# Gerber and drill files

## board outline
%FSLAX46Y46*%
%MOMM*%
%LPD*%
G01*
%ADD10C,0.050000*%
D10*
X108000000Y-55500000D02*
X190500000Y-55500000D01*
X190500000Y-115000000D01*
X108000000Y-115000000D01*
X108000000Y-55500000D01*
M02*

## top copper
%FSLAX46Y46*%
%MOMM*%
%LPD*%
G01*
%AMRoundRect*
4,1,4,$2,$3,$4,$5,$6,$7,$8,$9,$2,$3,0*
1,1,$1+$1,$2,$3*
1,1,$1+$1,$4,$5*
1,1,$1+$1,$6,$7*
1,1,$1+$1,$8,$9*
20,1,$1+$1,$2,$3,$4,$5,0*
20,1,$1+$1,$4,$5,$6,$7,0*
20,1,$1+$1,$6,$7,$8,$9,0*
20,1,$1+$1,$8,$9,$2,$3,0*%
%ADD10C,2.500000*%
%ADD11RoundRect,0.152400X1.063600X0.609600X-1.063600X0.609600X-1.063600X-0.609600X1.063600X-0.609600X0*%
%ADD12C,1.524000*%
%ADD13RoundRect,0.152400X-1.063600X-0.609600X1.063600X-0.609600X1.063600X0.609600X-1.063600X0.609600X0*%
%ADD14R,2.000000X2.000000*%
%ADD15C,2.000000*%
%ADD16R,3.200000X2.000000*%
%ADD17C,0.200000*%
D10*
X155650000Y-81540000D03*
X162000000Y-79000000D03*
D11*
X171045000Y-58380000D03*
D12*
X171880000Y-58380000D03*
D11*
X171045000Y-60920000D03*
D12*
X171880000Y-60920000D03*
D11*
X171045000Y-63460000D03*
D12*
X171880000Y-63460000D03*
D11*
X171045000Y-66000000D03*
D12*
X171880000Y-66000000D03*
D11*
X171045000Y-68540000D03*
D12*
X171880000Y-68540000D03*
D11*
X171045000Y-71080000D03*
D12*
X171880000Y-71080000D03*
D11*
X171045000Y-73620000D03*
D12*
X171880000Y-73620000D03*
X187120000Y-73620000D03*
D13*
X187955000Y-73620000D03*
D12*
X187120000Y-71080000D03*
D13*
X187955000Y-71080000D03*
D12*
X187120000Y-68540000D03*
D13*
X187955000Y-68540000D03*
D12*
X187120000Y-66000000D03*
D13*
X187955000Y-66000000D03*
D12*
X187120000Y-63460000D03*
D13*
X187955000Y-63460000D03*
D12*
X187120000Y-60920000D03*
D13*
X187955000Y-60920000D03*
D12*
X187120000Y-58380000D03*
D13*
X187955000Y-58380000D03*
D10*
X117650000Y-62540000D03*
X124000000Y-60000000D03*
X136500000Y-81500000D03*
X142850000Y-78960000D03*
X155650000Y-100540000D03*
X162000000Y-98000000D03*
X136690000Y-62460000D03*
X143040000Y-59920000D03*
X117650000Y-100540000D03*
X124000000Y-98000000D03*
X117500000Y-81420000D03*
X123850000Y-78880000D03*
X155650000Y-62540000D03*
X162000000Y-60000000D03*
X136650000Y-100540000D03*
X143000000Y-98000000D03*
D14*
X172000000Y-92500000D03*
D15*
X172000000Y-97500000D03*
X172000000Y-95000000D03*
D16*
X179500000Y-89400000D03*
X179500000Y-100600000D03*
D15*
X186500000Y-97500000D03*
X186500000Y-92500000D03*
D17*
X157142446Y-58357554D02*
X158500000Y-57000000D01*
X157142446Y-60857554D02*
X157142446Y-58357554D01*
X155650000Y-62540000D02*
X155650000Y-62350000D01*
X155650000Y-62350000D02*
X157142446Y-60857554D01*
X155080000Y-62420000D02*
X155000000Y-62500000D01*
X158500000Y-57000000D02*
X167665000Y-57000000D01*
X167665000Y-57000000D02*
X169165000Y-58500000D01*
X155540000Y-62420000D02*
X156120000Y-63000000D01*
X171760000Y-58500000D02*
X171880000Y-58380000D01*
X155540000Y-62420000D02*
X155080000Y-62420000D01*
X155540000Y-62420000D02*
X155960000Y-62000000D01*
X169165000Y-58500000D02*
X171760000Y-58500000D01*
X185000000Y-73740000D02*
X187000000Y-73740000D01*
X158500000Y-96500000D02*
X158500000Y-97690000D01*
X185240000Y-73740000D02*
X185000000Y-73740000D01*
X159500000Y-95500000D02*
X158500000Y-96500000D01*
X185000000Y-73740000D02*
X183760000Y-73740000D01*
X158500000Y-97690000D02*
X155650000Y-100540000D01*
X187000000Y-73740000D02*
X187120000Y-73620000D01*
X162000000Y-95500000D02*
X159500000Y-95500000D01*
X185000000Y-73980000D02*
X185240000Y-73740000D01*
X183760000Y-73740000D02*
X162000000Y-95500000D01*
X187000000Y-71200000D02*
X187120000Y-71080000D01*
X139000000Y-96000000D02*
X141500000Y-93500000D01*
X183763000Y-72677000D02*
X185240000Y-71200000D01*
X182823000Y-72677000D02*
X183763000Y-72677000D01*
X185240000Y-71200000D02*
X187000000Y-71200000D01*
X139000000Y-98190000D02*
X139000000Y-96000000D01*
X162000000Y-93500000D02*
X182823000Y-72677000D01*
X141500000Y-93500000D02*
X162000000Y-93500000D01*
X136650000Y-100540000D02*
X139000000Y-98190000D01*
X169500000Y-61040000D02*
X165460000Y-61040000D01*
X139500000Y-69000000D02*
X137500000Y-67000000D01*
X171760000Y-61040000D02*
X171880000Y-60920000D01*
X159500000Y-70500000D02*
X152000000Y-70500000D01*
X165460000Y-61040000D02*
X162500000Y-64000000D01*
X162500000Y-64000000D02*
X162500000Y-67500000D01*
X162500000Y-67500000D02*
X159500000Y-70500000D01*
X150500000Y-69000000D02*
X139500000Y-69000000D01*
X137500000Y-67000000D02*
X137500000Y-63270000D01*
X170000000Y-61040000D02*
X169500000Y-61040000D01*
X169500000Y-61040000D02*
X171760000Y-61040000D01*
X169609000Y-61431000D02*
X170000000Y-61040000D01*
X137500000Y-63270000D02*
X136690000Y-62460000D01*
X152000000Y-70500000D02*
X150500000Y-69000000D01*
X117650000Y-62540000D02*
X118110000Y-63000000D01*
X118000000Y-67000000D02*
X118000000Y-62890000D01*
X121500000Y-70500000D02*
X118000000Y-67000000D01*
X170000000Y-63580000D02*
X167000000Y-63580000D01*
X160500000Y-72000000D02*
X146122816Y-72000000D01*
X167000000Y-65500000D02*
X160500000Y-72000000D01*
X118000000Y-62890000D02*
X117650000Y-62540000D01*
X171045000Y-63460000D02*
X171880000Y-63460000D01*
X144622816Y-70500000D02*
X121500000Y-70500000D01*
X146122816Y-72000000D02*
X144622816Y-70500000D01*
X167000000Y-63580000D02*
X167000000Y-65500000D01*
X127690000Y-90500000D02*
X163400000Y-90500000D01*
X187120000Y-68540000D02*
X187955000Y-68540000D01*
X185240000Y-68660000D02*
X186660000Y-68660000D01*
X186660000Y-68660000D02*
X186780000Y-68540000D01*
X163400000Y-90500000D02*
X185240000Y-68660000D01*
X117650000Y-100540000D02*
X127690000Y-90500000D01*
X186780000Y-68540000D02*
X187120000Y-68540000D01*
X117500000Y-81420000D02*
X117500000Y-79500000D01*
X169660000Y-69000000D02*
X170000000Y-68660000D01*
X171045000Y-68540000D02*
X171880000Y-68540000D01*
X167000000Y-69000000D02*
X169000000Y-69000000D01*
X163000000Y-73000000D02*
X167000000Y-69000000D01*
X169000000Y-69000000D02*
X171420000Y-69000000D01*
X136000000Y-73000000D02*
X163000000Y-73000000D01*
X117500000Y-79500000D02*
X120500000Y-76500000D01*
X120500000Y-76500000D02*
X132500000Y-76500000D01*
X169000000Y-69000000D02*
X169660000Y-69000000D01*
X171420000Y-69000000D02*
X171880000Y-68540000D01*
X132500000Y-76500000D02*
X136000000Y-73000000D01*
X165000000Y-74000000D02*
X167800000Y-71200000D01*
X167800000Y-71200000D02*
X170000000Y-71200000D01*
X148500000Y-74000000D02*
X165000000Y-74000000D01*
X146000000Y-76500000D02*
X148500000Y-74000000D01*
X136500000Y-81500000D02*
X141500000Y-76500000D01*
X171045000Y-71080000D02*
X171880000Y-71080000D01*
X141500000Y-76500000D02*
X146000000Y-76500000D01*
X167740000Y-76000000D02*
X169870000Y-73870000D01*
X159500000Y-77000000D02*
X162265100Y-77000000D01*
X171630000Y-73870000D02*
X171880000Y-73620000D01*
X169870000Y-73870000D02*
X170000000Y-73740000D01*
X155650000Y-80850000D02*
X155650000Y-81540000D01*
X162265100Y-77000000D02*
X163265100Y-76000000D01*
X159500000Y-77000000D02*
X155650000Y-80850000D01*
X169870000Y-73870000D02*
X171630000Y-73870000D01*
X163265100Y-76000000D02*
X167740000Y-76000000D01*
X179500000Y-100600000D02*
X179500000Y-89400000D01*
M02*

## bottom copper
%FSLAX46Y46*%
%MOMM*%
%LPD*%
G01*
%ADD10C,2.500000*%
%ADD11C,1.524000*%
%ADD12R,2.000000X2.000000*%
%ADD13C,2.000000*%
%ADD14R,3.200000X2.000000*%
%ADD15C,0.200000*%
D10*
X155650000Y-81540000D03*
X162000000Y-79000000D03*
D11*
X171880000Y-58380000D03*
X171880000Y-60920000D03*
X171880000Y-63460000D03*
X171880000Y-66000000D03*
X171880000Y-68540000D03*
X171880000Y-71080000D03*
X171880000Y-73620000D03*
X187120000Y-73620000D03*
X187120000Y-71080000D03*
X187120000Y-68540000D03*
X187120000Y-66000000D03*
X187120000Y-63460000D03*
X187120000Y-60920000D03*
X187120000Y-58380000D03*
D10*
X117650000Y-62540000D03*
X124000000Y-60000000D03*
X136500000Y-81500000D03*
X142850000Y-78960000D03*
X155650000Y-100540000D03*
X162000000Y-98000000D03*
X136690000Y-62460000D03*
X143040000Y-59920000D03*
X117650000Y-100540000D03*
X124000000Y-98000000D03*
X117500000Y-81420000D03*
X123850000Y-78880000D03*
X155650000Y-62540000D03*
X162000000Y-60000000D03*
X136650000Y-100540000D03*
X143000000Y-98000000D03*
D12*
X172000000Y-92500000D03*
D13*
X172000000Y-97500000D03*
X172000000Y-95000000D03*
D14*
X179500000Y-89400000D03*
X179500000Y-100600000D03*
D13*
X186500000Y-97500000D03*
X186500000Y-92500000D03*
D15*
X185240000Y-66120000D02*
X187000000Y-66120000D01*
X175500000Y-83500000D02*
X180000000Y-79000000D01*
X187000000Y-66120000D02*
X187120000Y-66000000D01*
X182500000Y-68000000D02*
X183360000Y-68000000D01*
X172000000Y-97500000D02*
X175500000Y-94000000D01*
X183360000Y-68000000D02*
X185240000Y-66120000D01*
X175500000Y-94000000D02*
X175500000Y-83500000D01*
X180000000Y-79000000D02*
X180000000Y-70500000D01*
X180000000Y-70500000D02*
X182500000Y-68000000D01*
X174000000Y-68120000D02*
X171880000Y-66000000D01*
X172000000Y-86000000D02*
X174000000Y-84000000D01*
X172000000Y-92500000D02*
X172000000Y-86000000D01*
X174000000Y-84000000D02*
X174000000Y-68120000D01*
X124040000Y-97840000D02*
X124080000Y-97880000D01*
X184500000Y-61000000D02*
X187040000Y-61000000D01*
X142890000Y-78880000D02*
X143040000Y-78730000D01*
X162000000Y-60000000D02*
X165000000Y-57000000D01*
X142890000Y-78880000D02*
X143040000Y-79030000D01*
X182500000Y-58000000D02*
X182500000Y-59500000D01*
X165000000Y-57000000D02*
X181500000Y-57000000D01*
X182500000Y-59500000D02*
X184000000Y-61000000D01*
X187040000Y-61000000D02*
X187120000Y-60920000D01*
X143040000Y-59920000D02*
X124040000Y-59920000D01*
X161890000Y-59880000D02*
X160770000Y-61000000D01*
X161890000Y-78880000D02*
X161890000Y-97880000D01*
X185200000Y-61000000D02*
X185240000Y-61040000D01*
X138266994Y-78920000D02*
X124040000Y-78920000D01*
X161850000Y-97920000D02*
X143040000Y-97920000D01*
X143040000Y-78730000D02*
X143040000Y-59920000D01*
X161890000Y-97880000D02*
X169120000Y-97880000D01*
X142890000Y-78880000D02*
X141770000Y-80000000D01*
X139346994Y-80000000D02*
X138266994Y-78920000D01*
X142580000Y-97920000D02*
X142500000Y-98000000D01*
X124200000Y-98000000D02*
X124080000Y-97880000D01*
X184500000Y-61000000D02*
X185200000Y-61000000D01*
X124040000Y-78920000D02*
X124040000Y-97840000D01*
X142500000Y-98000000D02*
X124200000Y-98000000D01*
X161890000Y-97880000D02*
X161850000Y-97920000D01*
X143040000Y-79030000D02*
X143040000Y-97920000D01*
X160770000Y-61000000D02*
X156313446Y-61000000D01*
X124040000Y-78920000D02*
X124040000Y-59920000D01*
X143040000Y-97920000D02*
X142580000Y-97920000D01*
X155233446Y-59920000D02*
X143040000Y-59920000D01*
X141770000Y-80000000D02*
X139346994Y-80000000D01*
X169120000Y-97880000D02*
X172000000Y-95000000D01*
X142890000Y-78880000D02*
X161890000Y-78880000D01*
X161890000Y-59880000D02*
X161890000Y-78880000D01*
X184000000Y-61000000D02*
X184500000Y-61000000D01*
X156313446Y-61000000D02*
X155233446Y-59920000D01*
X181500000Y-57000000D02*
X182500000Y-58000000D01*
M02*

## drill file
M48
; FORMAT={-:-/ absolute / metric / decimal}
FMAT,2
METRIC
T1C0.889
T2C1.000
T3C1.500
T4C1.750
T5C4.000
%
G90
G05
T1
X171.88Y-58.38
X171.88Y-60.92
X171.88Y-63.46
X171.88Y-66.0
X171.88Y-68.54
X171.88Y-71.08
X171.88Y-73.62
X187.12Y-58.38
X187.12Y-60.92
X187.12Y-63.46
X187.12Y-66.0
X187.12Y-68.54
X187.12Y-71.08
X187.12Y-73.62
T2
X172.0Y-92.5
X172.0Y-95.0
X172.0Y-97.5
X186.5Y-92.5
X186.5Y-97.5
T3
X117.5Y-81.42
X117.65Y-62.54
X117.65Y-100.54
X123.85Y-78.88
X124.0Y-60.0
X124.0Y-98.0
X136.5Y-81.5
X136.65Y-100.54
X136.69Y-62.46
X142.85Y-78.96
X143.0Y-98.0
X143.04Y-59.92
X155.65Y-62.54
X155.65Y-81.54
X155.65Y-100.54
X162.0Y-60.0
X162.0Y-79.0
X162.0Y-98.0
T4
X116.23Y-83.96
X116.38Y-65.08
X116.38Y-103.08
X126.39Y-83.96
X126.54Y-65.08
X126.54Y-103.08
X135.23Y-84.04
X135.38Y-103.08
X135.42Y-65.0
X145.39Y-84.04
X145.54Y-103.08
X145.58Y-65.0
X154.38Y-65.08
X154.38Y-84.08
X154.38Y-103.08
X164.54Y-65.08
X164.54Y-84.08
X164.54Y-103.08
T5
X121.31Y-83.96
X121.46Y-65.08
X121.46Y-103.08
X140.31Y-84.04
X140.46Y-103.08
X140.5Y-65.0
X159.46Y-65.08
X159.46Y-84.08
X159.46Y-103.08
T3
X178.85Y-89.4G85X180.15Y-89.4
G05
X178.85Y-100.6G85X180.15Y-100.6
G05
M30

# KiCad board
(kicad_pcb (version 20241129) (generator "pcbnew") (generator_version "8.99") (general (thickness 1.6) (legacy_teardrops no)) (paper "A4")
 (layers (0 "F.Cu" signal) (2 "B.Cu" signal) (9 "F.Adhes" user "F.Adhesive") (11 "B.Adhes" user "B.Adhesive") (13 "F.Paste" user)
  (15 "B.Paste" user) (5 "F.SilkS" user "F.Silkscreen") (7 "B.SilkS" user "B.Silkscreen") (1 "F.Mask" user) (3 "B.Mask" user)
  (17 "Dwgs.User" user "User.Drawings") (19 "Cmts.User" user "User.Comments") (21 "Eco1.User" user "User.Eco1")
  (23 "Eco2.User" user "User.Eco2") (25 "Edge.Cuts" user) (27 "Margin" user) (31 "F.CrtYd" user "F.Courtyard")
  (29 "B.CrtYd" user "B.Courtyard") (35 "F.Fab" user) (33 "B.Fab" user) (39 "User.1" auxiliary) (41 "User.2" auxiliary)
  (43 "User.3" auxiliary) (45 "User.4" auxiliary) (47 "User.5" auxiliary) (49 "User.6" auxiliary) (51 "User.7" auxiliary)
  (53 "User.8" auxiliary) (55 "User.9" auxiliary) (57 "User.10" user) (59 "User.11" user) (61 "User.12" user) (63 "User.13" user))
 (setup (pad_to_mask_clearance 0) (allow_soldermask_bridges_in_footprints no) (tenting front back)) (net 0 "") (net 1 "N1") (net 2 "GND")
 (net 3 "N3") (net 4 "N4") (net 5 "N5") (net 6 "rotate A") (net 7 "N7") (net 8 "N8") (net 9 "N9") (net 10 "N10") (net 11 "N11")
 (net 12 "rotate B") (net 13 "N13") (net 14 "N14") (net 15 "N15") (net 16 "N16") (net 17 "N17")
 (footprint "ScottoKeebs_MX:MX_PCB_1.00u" (layer "F.Cu") (at 159.46 84.08)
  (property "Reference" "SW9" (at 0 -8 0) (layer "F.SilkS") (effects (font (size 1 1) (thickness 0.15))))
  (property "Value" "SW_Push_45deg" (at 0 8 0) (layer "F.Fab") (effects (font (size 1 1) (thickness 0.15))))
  (pad "" np_thru_hole circle (at -5.08 0) (size 1.75 1.75) (drill 1.75) (layers "*.Cu" "*.Mask"))
  (pad "" np_thru_hole circle (at 0 0) (size 4 4) (drill 4) (layers "*.Cu" "*.Mask"))
  (pad "" np_thru_hole circle (at 5.08 0) (size 1.75 1.75) (drill 1.75) (layers "*.Cu" "*.Mask"))
  (pad "1" thru_hole circle (at -3.81 -2.54) (size 2.5 2.5) (drill 1.5) (layers "*.Cu" "*.Mask") (remove_unused_layers no) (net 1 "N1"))
  (pad "2" thru_hole circle (at 2.54 -5.08) (size 2.5 2.5) (drill 1.5) (layers "*.Cu" "*.Mask") (remove_unused_layers no) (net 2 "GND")))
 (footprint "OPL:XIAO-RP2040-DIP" (layer "F.Cu") (at 179.5 66)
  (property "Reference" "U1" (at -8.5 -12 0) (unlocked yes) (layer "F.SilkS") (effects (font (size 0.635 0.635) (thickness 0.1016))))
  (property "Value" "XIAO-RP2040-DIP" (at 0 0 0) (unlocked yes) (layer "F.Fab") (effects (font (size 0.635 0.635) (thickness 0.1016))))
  (pad "1" smd roundrect (at -8.455 -7.62 180) (size 2.432 1.524) (layers "F.Cu" "F.Mask") (roundrect_rratio 0.1) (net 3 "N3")
   (thermal_bridge_angle 45))
  (pad "1" thru_hole circle (at -7.62 -7.62 180) (size 1.524 1.524) (drill 0.889) (layers "*.Cu" "*.Mask") (remove_unused_layers no)
   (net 3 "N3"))
  (pad "2" smd roundrect (at -8.455 -5.08 180) (size 2.432 1.524) (layers "F.Cu" "F.Mask") (roundrect_rratio 0.1) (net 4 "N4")
   (thermal_bridge_angle 45))
  (pad "2" thru_hole circle (at -7.62 -5.08 180) (size 1.524 1.524) (drill 0.889) (layers "*.Cu" "*.Mask") (remove_unused_layers no)
   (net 4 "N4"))
  (pad "3" smd roundrect (at -8.455 -2.54 180) (size 2.432 1.524) (layers "F.Cu" "F.Mask") (roundrect_rratio 0.1) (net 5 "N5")
   (thermal_bridge_angle 45))
  (pad "3" thru_hole circle (at -7.62 -2.54 180) (size 1.524 1.524) (drill 0.889) (layers "*.Cu" "*.Mask") (remove_unused_layers no)
   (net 5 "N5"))
  (pad "4" smd roundrect (at -8.455 0 180) (size 2.432 1.524) (layers "F.Cu" "F.Mask") (roundrect_rratio 0.1) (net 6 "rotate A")
   (thermal_bridge_angle 45))
  (pad "4" thru_hole circle (at -7.62 0 180) (size 1.524 1.524) (drill 0.889) (layers "*.Cu" "*.Mask") (remove_unused_layers no)
   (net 6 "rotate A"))
  (pad "5" smd roundrect (at -8.455 2.54 180) (size 2.432 1.524) (layers "F.Cu" "F.Mask") (roundrect_rratio 0.1) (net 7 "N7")
   (thermal_bridge_angle 45))
  (pad "5" thru_hole circle (at -7.62 2.54 180) (size 1.524 1.524) (drill 0.889) (layers "*.Cu" "*.Mask") (remove_unused_layers no)
   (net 7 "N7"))
  (pad "6" smd roundrect (at -8.455 5.08 180) (size 2.432 1.524) (layers "F.Cu" "F.Mask") (roundrect_rratio 0.1) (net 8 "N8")
   (thermal_bridge_angle 45))
  (pad "6" thru_hole circle (at -7.62 5.08 180) (size 1.524 1.524) (drill 0.889) (layers "*.Cu" "*.Mask") (remove_unused_layers no)
   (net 8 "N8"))
  (pad "7" smd roundrect (at -8.455 7.62 180) (size 2.432 1.524) (layers "F.Cu" "F.Mask") (roundrect_rratio 0.1) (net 1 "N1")
   (thermal_bridge_angle 45))
  (pad "7" thru_hole circle (at -7.62 7.62 180) (size 1.524 1.524) (drill 0.889) (layers "*.Cu" "*.Mask") (remove_unused_layers no)
   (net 1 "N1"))
  (pad "8" thru_hole circle (at 7.62 7.62) (size 1.524 1.524) (drill 0.889) (layers "*.Cu" "*.Mask") (remove_unused_layers no) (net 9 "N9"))
  (pad "8" smd roundrect (at 8.455 7.62) (size 2.432 1.524) (layers "F.Cu" "F.Mask") (roundrect_rratio 0.1) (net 9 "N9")
   (thermal_bridge_angle 45))
  (pad "9" thru_hole circle (at 7.62 5.08) (size 1.524 1.524) (drill 0.889) (layers "*.Cu" "*.Mask") (remove_unused_layers no)
   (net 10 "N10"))
  (pad "9" smd roundrect (at 8.455 5.08) (size 2.432 1.524) (layers "F.Cu" "F.Mask") (roundrect_rratio 0.1) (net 10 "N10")
   (thermal_bridge_angle 45))
  (pad "10" thru_hole circle (at 7.62 2.54) (size 1.524 1.524) (drill 0.889) (layers "*.Cu" "*.Mask") (remove_unused_layers no)
   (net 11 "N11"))
  (pad "10" smd roundrect (at 8.455 2.54) (size 2.432 1.524) (layers "F.Cu" "F.Mask") (roundrect_rratio 0.1) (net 11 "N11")
   (thermal_bridge_angle 45))
  (pad "11" thru_hole circle (at 7.62 0) (size 1.524 1.524) (drill 0.889) (layers "*.Cu" "*.Mask") (remove_unused_layers no)
   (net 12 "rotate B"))
  (pad "11" smd roundrect (at 8.455 0) (size 2.432 1.524) (layers "F.Cu" "F.Mask") (roundrect_rratio 0.1) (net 12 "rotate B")
   (thermal_bridge_angle 45))
  (pad "12" thru_hole circle (at 7.62 -2.54) (size 1.524 1.524) (drill 0.889) (layers "*.Cu" "*.Mask") (remove_unused_layers no)
   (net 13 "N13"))
  (pad "12" smd roundrect (at 8.455 -2.54) (size 2.432 1.524) (layers "F.Cu" "F.Mask") (roundrect_rratio 0.1) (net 13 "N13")
   (thermal_bridge_angle 45))
  (pad "13" thru_hole circle (at 7.62 -5.08) (size 1.524 1.524) (drill 0.889) (layers "*.Cu" "*.Mask") (remove_unused_layers no)
   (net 2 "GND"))
  (pad "13" smd roundrect (at 8.455 -5.08) (size 2.432 1.524) (layers "F.Cu" "F.Mask") (roundrect_rratio 0.1) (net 2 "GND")
   (thermal_bridge_angle 45))
  (pad "14" thru_hole circle (at 7.62 -7.62) (size 1.524 1.524) (drill 0.889) (layers "*.Cu" "*.Mask") (remove_unused_layers no)
   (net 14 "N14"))
  (pad "14" smd roundrect (at 8.455 -7.62) (size 2.432 1.524) (layers "F.Cu" "F.Mask") (roundrect_rratio 0.1) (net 14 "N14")
   (thermal_bridge_angle 45)))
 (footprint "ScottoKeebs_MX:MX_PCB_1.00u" (layer "F.Cu") (at 121.46 65.08)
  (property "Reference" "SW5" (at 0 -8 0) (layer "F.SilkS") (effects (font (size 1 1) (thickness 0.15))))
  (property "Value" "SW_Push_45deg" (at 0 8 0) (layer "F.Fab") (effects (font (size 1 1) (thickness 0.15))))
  (pad "" np_thru_hole circle (at -5.08 0) (size 1.75 1.75) (drill 1.75) (layers "*.Cu" "*.Mask"))
  (pad "" np_thru_hole circle (at 0 0) (size 4 4) (drill 4) (layers "*.Cu" "*.Mask"))
  (pad "" np_thru_hole circle (at 5.08 0) (size 1.75 1.75) (drill 1.75) (layers "*.Cu" "*.Mask"))
  (pad "1" thru_hole circle (at -3.81 -2.54) (size 2.5 2.5) (drill 1.5) (layers "*.Cu" "*.Mask") (remove_unused_layers no) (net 5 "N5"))
  (pad "2" thru_hole circle (at 2.54 -5.08) (size 2.5 2.5) (drill 1.5) (layers "*.Cu" "*.Mask") (remove_unused_layers no) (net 2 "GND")))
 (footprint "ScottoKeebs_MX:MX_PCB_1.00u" (layer "F.Cu") (at 140.31 84.04)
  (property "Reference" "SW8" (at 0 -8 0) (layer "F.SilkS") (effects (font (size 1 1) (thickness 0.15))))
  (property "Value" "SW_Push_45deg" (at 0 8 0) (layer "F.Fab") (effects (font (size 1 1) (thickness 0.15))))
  (pad "" np_thru_hole circle (at -5.08 0) (size 1.75 1.75) (drill 1.75) (layers "*.Cu" "*.Mask"))
  (pad "" np_thru_hole circle (at 0 0) (size 4 4) (drill 4) (layers "*.Cu" "*.Mask"))
  (pad "" np_thru_hole circle (at 5.08 0) (size 1.75 1.75) (drill 1.75) (layers "*.Cu" "*.Mask"))
  (pad "1" thru_hole circle (at -3.81 -2.54) (size 2.5 2.5) (drill 1.5) (layers "*.Cu" "*.Mask") (remove_unused_layers no) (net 8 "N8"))
  (pad "2" thru_hole circle (at 2.54 -5.08) (size 2.5 2.5) (drill 1.5) (layers "*.Cu" "*.Mask") (remove_unused_layers no) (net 2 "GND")))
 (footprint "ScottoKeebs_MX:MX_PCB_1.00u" (layer "F.Cu") (at 159.46 103.08)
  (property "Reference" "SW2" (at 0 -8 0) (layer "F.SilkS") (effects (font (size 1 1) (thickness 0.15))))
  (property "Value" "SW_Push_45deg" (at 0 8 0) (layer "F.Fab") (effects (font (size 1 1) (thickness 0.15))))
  (pad "" np_thru_hole circle (at -5.08 0) (size 1.75 1.75) (drill 1.75) (layers "*.Cu" "*.Mask"))
  (pad "" np_thru_hole circle (at 0 0) (size 4 4) (drill 4) (layers "*.Cu" "*.Mask"))
  (pad "" np_thru_hole circle (at 5.08 0) (size 1.75 1.75) (drill 1.75) (layers "*.Cu" "*.Mask"))
  (pad "1" thru_hole circle (at -3.81 -2.54) (size 2.5 2.5) (drill 1.5) (layers "*.Cu" "*.Mask") (remove_unused_layers no) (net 9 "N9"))
  (pad "2" thru_hole circle (at 2.54 -5.08) (size 2.5 2.5) (drill 1.5) (layers "*.Cu" "*.Mask") (remove_unused_layers no) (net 2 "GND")))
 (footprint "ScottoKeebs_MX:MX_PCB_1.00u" (layer "F.Cu") (at 140.5 65)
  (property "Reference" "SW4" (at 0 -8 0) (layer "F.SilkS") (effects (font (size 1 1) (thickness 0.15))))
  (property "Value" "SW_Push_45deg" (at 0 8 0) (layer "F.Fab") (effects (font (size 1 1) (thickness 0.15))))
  (pad "" np_thru_hole circle (at -5.08 0) (size 1.75 1.75) (drill 1.75) (layers "*.Cu" "*.Mask"))
  (pad "" np_thru_hole circle (at 0 0) (size 4 4) (drill 4) (layers "*.Cu" "*.Mask"))
  (pad "" np_thru_hole circle (at 5.08 0) (size 1.75 1.75) (drill 1.75) (layers "*.Cu" "*.Mask"))
  (pad "1" thru_hole circle (at -3.81 -2.54) (size 2.5 2.5) (drill 1.5) (layers "*.Cu" "*.Mask") (remove_unused_layers no) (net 4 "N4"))
  (pad "2" thru_hole circle (at 2.54 -5.08) (size 2.5 2.5) (drill 1.5) (layers "*.Cu" "*.Mask") (remove_unused_layers no) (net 2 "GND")))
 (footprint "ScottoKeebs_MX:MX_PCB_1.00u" (layer "F.Cu") (at 121.46 103.08)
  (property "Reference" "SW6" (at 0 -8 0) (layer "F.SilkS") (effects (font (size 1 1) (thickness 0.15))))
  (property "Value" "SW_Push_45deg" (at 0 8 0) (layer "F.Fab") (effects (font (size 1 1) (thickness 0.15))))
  (pad "" np_thru_hole circle (at -5.08 0) (size 1.75 1.75) (drill 1.75) (layers "*.Cu" "*.Mask"))
  (pad "" np_thru_hole circle (at 0 0) (size 4 4) (drill 4) (layers "*.Cu" "*.Mask"))
  (pad "" np_thru_hole circle (at 5.08 0) (size 1.75 1.75) (drill 1.75) (layers "*.Cu" "*.Mask"))
  (pad "1" thru_hole circle (at -3.81 -2.54) (size 2.5 2.5) (drill 1.5) (layers "*.Cu" "*.Mask") (remove_unused_layers no) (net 11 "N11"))
  (pad "2" thru_hole circle (at 2.54 -5.08) (size 2.5 2.5) (drill 1.5) (layers "*.Cu" "*.Mask") (remove_unused_layers no) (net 2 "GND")))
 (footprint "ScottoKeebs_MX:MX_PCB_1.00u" (layer "F.Cu") (at 121.31 83.96)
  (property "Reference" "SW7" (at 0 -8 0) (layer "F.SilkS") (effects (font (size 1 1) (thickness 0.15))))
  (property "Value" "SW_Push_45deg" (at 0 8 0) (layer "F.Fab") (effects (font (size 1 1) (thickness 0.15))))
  (pad "" np_thru_hole circle (at -5.08 0) (size 1.75 1.75) (drill 1.75) (layers "*.Cu" "*.Mask"))
  (pad "" np_thru_hole circle (at 0 0) (size 4 4) (drill 4) (layers "*.Cu" "*.Mask"))
  (pad "" np_thru_hole circle (at 5.08 0) (size 1.75 1.75) (drill 1.75) (layers "*.Cu" "*.Mask"))
  (pad "1" thru_hole circle (at -3.81 -2.54) (size 2.5 2.5) (drill 1.5) (layers "*.Cu" "*.Mask") (remove_unused_layers no) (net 7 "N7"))
  (pad "2" thru_hole circle (at 2.54 -5.08) (size 2.5 2.5) (drill 1.5) (layers "*.Cu" "*.Mask") (remove_unused_layers no) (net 2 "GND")))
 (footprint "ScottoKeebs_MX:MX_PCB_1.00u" (layer "F.Cu") (at 159.46 65.08)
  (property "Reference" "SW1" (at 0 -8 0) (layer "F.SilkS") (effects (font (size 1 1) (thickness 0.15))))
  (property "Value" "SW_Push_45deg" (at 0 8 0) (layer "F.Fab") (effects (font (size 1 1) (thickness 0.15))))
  (pad "" np_thru_hole circle (at -5.08 0) (size 1.75 1.75) (drill 1.75) (layers "*.Cu" "*.Mask"))
  (pad "" np_thru_hole circle (at 0 0) (size 4 4) (drill 4) (layers "*.Cu" "*.Mask"))
  (pad "" np_thru_hole circle (at 5.08 0) (size 1.75 1.75) (drill 1.75) (layers "*.Cu" "*.Mask"))
  (pad "1" thru_hole circle (at -3.81 -2.54) (size 2.5 2.5) (drill 1.5) (layers "*.Cu" "*.Mask") (remove_unused_layers no) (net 3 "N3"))
  (pad "2" thru_hole circle (at 2.54 -5.08) (size 2.5 2.5) (drill 1.5) (layers "*.Cu" "*.Mask") (remove_unused_layers no) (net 2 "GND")))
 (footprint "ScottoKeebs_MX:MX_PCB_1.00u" (layer "F.Cu") (at 140.46 103.08)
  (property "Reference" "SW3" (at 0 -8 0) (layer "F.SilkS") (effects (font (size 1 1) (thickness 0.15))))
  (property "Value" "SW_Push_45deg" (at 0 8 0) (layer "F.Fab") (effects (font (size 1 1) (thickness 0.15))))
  (pad "" np_thru_hole circle (at -5.08 0) (size 1.75 1.75) (drill 1.75) (layers "*.Cu" "*.Mask"))
  (pad "" np_thru_hole circle (at 0 0) (size 4 4) (drill 4) (layers "*.Cu" "*.Mask"))
  (pad "" np_thru_hole circle (at 5.08 0) (size 1.75 1.75) (drill 1.75) (layers "*.Cu" "*.Mask"))
  (pad "1" thru_hole circle (at -3.81 -2.54) (size 2.5 2.5) (drill 1.5) (layers "*.Cu" "*.Mask") (remove_unused_layers no) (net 10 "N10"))
  (pad "2" thru_hole circle (at 2.54 -5.08) (size 2.5 2.5) (drill 1.5) (layers "*.Cu" "*.Mask") (remove_unused_layers no) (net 2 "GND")))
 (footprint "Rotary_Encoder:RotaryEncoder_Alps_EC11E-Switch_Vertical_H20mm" (layer "F.Cu") (at 172 92.5)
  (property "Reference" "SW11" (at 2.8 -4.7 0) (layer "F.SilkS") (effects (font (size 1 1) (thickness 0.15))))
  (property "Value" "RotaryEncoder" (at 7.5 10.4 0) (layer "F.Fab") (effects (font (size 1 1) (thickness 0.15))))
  (pad "A" thru_hole rect (at 0 0) (size 2 2) (drill 1) (layers "*.Cu" "*.Mask") (remove_unused_layers no) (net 6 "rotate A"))
  (pad "B" thru_hole circle (at 0 5) (size 2 2) (drill 1) (layers "*.Cu" "*.Mask") (remove_unused_layers no) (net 12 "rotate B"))
  (pad "C" thru_hole circle (at 0 2.5) (size 2 2) (drill 1) (layers "*.Cu" "*.Mask") (remove_unused_layers no) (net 2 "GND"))
  (pad "MP" thru_hole rect (at 7.5 -3.1) (size 3.2 2) (drill oval 2.8 1.5) (layers "*.Cu" "*.Mask") (remove_unused_layers no) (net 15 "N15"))
  (pad "MP" thru_hole rect (at 7.5 8.1) (size 3.2 2) (drill oval 2.8 1.5) (layers "*.Cu" "*.Mask") (remove_unused_layers no) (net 15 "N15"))
  (pad "S1" thru_hole circle (at 14.5 5) (size 2 2) (drill 1) (layers "*.Cu" "*.Mask") (remove_unused_layers no) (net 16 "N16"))
  (pad "S2" thru_hole circle (at 14.5 0) (size 2 2) (drill 1) (layers "*.Cu" "*.Mask") (remove_unused_layers no) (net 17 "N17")))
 (gr_rect (start 108 55.5) (end 190.5 115) (stroke (width 0.05) (type default)) (fill no) (layer "Edge.Cuts"))
 (segment (start 157.142446 58.357554) (end 158.5 57) (width 0.2) (layer "F.Cu") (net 3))
 (segment (start 157.142446 60.857554) (end 157.142446 58.357554) (width 0.2) (layer "F.Cu") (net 3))
 (segment (start 155.65 62.54) (end 155.65 62.35) (width 0.2) (layer "F.Cu") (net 3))
 (segment (start 155.65 62.35) (end 157.142446 60.857554) (width 0.2) (layer "F.Cu") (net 3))
 (segment (start 155.08 62.42) (end 155 62.5) (width 0.2) (layer "F.Cu") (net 3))
 (segment (start 158.5 57) (end 167.665 57) (width 0.2) (layer "F.Cu") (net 3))
 (segment (start 167.665 57) (end 169.165 58.5) (width 0.2) (layer "F.Cu") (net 3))
 (segment (start 155.54 62.42) (end 156.12 63) (width 0.2) (layer "F.Cu") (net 3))
 (segment (start 171.76 58.5) (end 171.88 58.38) (width 0.2) (layer "F.Cu") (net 3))
 (segment (start 155.54 62.42) (end 155.08 62.42) (width 0.2) (layer "F.Cu") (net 3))
 (segment (start 155.54 62.42) (end 155.96 62) (width 0.2) (layer "F.Cu") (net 3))
 (segment (start 169.165 58.5) (end 171.76 58.5) (width 0.2) (layer "F.Cu") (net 3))
 (segment (start 185 73.74) (end 187 73.74) (width 0.2) (layer "F.Cu") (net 9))
 (segment (start 158.5 96.5) (end 158.5 97.69) (width 0.2) (layer "F.Cu") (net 9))
 (segment (start 185.24 73.74) (end 185 73.74) (width 0.2) (layer "F.Cu") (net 9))
 (segment (start 159.5 95.5) (end 158.5 96.5) (width 0.2) (layer "F.Cu") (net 9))
 (segment (start 185 73.74) (end 183.76 73.74) (width 0.2) (layer "F.Cu") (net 9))
 (segment (start 158.5 97.69) (end 155.65 100.54) (width 0.2) (layer "F.Cu") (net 9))
 (segment (start 187 73.74) (end 187.12 73.62) (width 0.2) (layer "F.Cu") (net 9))
 (segment (start 162 95.5) (end 159.5 95.5) (width 0.2) (layer "F.Cu") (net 9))
 (segment (start 185 73.98) (end 185.24 73.74) (width 0.2) (layer "F.Cu") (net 9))
 (segment (start 183.76 73.74) (end 162 95.5) (width 0.2) (layer "F.Cu") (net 9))
 (segment (start 187 71.2) (end 187.12 71.08) (width 0.2) (layer "F.Cu") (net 10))
 (segment (start 139 96) (end 141.5 93.5) (width 0.2) (layer "F.Cu") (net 10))
 (segment (start 183.763 72.677) (end 185.24 71.2) (width 0.2) (layer "F.Cu") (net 10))
 (segment (start 182.823 72.677) (end 183.763 72.677) (width 0.2) (layer "F.Cu") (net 10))
 (segment (start 185.24 71.2) (end 187 71.2) (width 0.2) (layer "F.Cu") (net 10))
 (segment (start 139 98.19) (end 139 96) (width 0.2) (layer "F.Cu") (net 10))
 (segment (start 162 93.5) (end 182.823 72.677) (width 0.2) (layer "F.Cu") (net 10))
 (segment (start 141.5 93.5) (end 162 93.5) (width 0.2) (layer "F.Cu") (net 10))
 (segment (start 136.65 100.54) (end 139 98.19) (width 0.2) (layer "F.Cu") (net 10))
 (segment (start 169.5 61.04) (end 165.46 61.04) (width 0.2) (layer "F.Cu") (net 4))
 (segment (start 139.5 69) (end 137.5 67) (width 0.2) (layer "F.Cu") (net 4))
 (segment (start 171.76 61.04) (end 171.88 60.92) (width 0.2) (layer "F.Cu") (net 4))
 (segment (start 159.5 70.5) (end 152 70.5) (width 0.2) (layer "F.Cu") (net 4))
 (segment (start 165.46 61.04) (end 162.5 64) (width 0.2) (layer "F.Cu") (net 4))
 (segment (start 162.5 64) (end 162.5 67.5) (width 0.2) (layer "F.Cu") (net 4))
 (segment (start 162.5 67.5) (end 159.5 70.5) (width 0.2) (layer "F.Cu") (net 4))
 (segment (start 150.5 69) (end 139.5 69) (width 0.2) (layer "F.Cu") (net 4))
 (segment (start 137.5 67) (end 137.5 63.27) (width 0.2) (layer "F.Cu") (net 4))
 (segment (start 170 61.04) (end 169.5 61.04) (width 0.2) (layer "F.Cu") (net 4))
 (segment (start 169.5 61.04) (end 171.76 61.04) (width 0.2) (layer "F.Cu") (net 4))
 (segment (start 169.609 61.431) (end 170 61.04) (width 0.2) (layer "F.Cu") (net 4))
 (segment (start 137.5 63.27) (end 136.69 62.46) (width 0.2) (layer "F.Cu") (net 4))
 (segment (start 152 70.5) (end 150.5 69) (width 0.2) (layer "F.Cu") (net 4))
 (segment (start 117.65 62.54) (end 118.11 63) (width 0.2) (layer "F.Cu") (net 5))
 (segment (start 118 67) (end 118 62.89) (width 0.2) (layer "F.Cu") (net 5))
 (segment (start 121.5 70.5) (end 118 67) (width 0.2) (layer "F.Cu") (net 5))
 (segment (start 170 63.58) (end 167 63.58) (width 0.2) (layer "F.Cu") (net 5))
 (segment (start 160.5 72) (end 146.122816 72) (width 0.2) (layer "F.Cu") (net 5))
 (segment (start 167 65.5) (end 160.5 72) (width 0.2) (layer "F.Cu") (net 5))
 (segment (start 118 62.89) (end 117.65 62.54) (width 0.2) (layer "F.Cu") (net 5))
 (segment (start 171.045 63.46) (end 171.88 63.46) (width 0.2) (layer "F.Cu") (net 5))
 (segment (start 144.622816 70.5) (end 121.5 70.5) (width 0.2) (layer "F.Cu") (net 5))
 (segment (start 146.122816 72) (end 144.622816 70.5) (width 0.2) (layer "F.Cu") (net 5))
 (segment (start 167 63.58) (end 167 65.5) (width 0.2) (layer "F.Cu") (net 5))
 (segment (start 127.69 90.5) (end 163.4 90.5) (width 0.2) (layer "F.Cu") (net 11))
 (segment (start 187.12 68.54) (end 187.955 68.54) (width 0.2) (layer "F.Cu") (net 11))
 (segment (start 185.24 68.66) (end 186.66 68.66) (width 0.2) (layer "F.Cu") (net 11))
 (segment (start 186.66 68.66) (end 186.78 68.54) (width 0.2) (layer "F.Cu") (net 11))
 (segment (start 163.4 90.5) (end 185.24 68.66) (width 0.2) (layer "F.Cu") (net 11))
 (segment (start 117.65 100.54) (end 127.69 90.5) (width 0.2) (layer "F.Cu") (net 11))
 (segment (start 186.78 68.54) (end 187.12 68.54) (width 0.2) (layer "F.Cu") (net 11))
 (segment (start 117.5 81.42) (end 117.5 79.5) (width 0.2) (layer "F.Cu") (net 7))
 (segment (start 169.66 69) (end 170 68.66) (width 0.2) (layer "F.Cu") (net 7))
 (segment (start 171.045 68.54) (end 171.88 68.54) (width 0.2) (layer "F.Cu") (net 7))
 (segment (start 167 69) (end 169 69) (width 0.2) (layer "F.Cu") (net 7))
 (segment (start 163 73) (end 167 69) (width 0.2) (layer "F.Cu") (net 7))
 (segment (start 169 69) (end 171.42 69) (width 0.2) (layer "F.Cu") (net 7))
 (segment (start 136 73) (end 163 73) (width 0.2) (layer "F.Cu") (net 7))
 (segment (start 117.5 79.5) (end 120.5 76.5) (width 0.2) (layer "F.Cu") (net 7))
 (segment (start 120.5 76.5) (end 132.5 76.5) (width 0.2) (layer "F.Cu") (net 7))
 (segment (start 169 69) (end 169.66 69) (width 0.2) (layer "F.Cu") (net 7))
 (segment (start 171.42 69) (end 171.88 68.54) (width 0.2) (layer "F.Cu") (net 7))
 (segment (start 132.5 76.5) (end 136 73) (width 0.2) (layer "F.Cu") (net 7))
 (segment (start 165 74) (end 167.8 71.2) (width 0.2) (layer "F.Cu") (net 8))
 (segment (start 167.8 71.2) (end 170 71.2) (width 0.2) (layer "F.Cu") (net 8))
 (segment (start 148.5 74) (end 165 74) (width 0.2) (layer "F.Cu") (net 8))
 (segment (start 146 76.5) (end 148.5 74) (width 0.2) (layer "F.Cu") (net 8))
 (segment (start 136.5 81.5) (end 141.5 76.5) (width 0.2) (layer "F.Cu") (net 8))
 (segment (start 171.045 71.08) (end 171.88 71.08) (width 0.2) (layer "F.Cu") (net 8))
 (segment (start 141.5 76.5) (end 146 76.5) (width 0.2) (layer "F.Cu") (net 8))
 (segment (start 167.74 76) (end 169.87 73.87) (width 0.2) (layer "F.Cu") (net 1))
 (segment (start 159.5 77) (end 162.2651 77) (width 0.2) (layer "F.Cu") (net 1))
 (segment (start 171.63 73.87) (end 171.88 73.62) (width 0.2) (layer "F.Cu") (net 1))
 (segment (start 169.87 73.87) (end 170 73.74) (width 0.2) (layer "F.Cu") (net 1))
 (segment (start 155.65 80.85) (end 155.65 81.54) (width 0.2) (layer "F.Cu") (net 1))
 (segment (start 162.2651 77) (end 163.2651 76) (width 0.2) (layer "F.Cu") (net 1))
 (segment (start 159.5 77) (end 155.65 80.85) (width 0.2) (layer "F.Cu") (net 1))
 (segment (start 169.87 73.87) (end 171.63 73.87) (width 0.2) (layer "F.Cu") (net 1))
 (segment (start 163.2651 76) (end 167.74 76) (width 0.2) (layer "F.Cu") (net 1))
 (segment (start 185.24 66.12) (end 187 66.12) (width 0.2) (layer "B.Cu") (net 12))
 (segment (start 175.5 83.5) (end 180 79) (width 0.2) (layer "B.Cu") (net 12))
 (segment (start 187 66.12) (end 187.12 66) (width 0.2) (layer "B.Cu") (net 12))
 (segment (start 182.5 68) (end 183.36 68) (width 0.2) (layer "B.Cu") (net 12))
 (segment (start 172 97.5) (end 175.5 94) (width 0.2) (layer "B.Cu") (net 12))
 (segment (start 183.36 68) (end 185.24 66.12) (width 0.2) (layer "B.Cu") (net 12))
 (segment (start 175.5 94) (end 175.5 83.5) (width 0.2) (layer "B.Cu") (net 12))
 (segment (start 180 79) (end 180 70.5) (width 0.2) (layer "B.Cu") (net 12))
 (segment (start 180 70.5) (end 182.5 68) (width 0.2) (layer "B.Cu") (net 12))
 (segment (start 174 68.12) (end 171.88 66) (width 0.2) (layer "B.Cu") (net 6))
 (segment (start 172 86) (end 174 84) (width 0.2) (layer "B.Cu") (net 6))
 (segment (start 172 92.5) (end 172 86) (width 0.2) (layer "B.Cu") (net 6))
 (segment (start 174 84) (end 174 68.12) (width 0.2) (layer "B.Cu") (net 6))
 (segment (start 124.04 97.84) (end 124.08 97.88) (width 0.2) (layer "B.Cu") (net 2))
 (segment (start 184.5 61) (end 187.04 61) (width 0.2) (layer "B.Cu") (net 2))
 (segment (start 142.89 78.88) (end 143.04 78.73) (width 0.2) (layer "B.Cu") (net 2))
 (segment (start 162 60) (end 165 57) (width 0.2) (layer "B.Cu") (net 2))
 (segment (start 142.89 78.88) (end 143.04 79.03) (width 0.2) (layer "B.Cu") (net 2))
 (segment (start 182.5 58) (end 182.5 59.5) (width 0.2) (layer "B.Cu") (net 2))
 (segment (start 165 57) (end 181.5 57) (width 0.2) (layer "B.Cu") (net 2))
 (segment (start 182.5 59.5) (end 184 61) (width 0.2) (layer "B.Cu") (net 2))
 (segment (start 187.04 61) (end 187.12 60.92) (width 0.2) (layer "B.Cu") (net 2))
 (segment (start 143.04 59.92) (end 124.04 59.92) (width 0.2) (layer "B.Cu") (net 2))
 (segment (start 161.89 59.88) (end 160.77 61) (width 0.2) (layer "B.Cu") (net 2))
 (segment (start 161.89 78.88) (end 161.89 97.88) (width 0.2) (layer "B.Cu") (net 2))
 (segment (start 185.2 61) (end 185.24 61.04) (width 0.2) (layer "B.Cu") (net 2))
 (segment (start 138.266994 78.92) (end 124.04 78.92) (width 0.2) (layer "B.Cu") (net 2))
 (segment (start 161.85 97.92) (end 143.04 97.92) (width 0.2) (layer "B.Cu") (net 2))
 (segment (start 143.04 78.73) (end 143.04 59.92) (width 0.2) (layer "B.Cu") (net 2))
 (segment (start 161.89 97.88) (end 169.12 97.88) (width 0.2) (layer "B.Cu") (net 2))
 (segment (start 142.89 78.88) (end 141.77 80) (width 0.2) (layer "B.Cu") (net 2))
 (segment (start 139.346994 80) (end 138.266994 78.92) (width 0.2) (layer "B.Cu") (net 2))
 (segment (start 142.58 97.92) (end 142.5 98) (width 0.2) (layer "B.Cu") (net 2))
 (segment (start 124.2 98) (end 124.08 97.88) (width 0.2) (layer "B.Cu") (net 2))
 (segment (start 184.5 61) (end 185.2 61) (width 0.2) (layer "B.Cu") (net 2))
 (segment (start 124.04 78.92) (end 124.04 97.84) (width 0.2) (layer "B.Cu") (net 2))
 (segment (start 142.5 98) (end 124.2 98) (width 0.2) (layer "B.Cu") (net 2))
 (segment (start 161.89 97.88) (end 161.85 97.92) (width 0.2) (layer "B.Cu") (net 2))
 (segment (start 143.04 79.03) (end 143.04 97.92) (width 0.2) (layer "B.Cu") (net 2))
 (segment (start 160.77 61) (end 156.313446 61) (width 0.2) (layer "B.Cu") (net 2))
 (segment (start 124.04 78.92) (end 124.04 59.92) (width 0.2) (layer "B.Cu") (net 2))
 (segment (start 143.04 97.92) (end 142.58 97.92) (width 0.2) (layer "B.Cu") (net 2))
 (segment (start 155.233446 59.92) (end 143.04 59.92) (width 0.2) (layer "B.Cu") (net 2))
 (segment (start 141.77 80) (end 139.346994 80) (width 0.2) (layer "B.Cu") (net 2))
 (segment (start 169.12 97.88) (end 172 95) (width 0.2) (layer "B.Cu") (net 2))
 (segment (start 142.89 78.88) (end 161.89 78.88) (width 0.2) (layer "B.Cu") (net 2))
 (segment (start 161.89 59.88) (end 161.89 78.88) (width 0.2) (layer "B.Cu") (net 2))
 (segment (start 184 61) (end 184.5 61) (width 0.2) (layer "B.Cu") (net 2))
 (segment (start 156.313446 61) (end 155.233446 59.92) (width 0.2) (layer "B.Cu") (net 2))
 (segment (start 181.5 57) (end 182.5 58) (width 0.2) (layer "B.Cu") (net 2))
 (segment (start 179.5 100.6) (end 179.5 89.4) (width 0.2) (layer "F.Cu") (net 15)))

